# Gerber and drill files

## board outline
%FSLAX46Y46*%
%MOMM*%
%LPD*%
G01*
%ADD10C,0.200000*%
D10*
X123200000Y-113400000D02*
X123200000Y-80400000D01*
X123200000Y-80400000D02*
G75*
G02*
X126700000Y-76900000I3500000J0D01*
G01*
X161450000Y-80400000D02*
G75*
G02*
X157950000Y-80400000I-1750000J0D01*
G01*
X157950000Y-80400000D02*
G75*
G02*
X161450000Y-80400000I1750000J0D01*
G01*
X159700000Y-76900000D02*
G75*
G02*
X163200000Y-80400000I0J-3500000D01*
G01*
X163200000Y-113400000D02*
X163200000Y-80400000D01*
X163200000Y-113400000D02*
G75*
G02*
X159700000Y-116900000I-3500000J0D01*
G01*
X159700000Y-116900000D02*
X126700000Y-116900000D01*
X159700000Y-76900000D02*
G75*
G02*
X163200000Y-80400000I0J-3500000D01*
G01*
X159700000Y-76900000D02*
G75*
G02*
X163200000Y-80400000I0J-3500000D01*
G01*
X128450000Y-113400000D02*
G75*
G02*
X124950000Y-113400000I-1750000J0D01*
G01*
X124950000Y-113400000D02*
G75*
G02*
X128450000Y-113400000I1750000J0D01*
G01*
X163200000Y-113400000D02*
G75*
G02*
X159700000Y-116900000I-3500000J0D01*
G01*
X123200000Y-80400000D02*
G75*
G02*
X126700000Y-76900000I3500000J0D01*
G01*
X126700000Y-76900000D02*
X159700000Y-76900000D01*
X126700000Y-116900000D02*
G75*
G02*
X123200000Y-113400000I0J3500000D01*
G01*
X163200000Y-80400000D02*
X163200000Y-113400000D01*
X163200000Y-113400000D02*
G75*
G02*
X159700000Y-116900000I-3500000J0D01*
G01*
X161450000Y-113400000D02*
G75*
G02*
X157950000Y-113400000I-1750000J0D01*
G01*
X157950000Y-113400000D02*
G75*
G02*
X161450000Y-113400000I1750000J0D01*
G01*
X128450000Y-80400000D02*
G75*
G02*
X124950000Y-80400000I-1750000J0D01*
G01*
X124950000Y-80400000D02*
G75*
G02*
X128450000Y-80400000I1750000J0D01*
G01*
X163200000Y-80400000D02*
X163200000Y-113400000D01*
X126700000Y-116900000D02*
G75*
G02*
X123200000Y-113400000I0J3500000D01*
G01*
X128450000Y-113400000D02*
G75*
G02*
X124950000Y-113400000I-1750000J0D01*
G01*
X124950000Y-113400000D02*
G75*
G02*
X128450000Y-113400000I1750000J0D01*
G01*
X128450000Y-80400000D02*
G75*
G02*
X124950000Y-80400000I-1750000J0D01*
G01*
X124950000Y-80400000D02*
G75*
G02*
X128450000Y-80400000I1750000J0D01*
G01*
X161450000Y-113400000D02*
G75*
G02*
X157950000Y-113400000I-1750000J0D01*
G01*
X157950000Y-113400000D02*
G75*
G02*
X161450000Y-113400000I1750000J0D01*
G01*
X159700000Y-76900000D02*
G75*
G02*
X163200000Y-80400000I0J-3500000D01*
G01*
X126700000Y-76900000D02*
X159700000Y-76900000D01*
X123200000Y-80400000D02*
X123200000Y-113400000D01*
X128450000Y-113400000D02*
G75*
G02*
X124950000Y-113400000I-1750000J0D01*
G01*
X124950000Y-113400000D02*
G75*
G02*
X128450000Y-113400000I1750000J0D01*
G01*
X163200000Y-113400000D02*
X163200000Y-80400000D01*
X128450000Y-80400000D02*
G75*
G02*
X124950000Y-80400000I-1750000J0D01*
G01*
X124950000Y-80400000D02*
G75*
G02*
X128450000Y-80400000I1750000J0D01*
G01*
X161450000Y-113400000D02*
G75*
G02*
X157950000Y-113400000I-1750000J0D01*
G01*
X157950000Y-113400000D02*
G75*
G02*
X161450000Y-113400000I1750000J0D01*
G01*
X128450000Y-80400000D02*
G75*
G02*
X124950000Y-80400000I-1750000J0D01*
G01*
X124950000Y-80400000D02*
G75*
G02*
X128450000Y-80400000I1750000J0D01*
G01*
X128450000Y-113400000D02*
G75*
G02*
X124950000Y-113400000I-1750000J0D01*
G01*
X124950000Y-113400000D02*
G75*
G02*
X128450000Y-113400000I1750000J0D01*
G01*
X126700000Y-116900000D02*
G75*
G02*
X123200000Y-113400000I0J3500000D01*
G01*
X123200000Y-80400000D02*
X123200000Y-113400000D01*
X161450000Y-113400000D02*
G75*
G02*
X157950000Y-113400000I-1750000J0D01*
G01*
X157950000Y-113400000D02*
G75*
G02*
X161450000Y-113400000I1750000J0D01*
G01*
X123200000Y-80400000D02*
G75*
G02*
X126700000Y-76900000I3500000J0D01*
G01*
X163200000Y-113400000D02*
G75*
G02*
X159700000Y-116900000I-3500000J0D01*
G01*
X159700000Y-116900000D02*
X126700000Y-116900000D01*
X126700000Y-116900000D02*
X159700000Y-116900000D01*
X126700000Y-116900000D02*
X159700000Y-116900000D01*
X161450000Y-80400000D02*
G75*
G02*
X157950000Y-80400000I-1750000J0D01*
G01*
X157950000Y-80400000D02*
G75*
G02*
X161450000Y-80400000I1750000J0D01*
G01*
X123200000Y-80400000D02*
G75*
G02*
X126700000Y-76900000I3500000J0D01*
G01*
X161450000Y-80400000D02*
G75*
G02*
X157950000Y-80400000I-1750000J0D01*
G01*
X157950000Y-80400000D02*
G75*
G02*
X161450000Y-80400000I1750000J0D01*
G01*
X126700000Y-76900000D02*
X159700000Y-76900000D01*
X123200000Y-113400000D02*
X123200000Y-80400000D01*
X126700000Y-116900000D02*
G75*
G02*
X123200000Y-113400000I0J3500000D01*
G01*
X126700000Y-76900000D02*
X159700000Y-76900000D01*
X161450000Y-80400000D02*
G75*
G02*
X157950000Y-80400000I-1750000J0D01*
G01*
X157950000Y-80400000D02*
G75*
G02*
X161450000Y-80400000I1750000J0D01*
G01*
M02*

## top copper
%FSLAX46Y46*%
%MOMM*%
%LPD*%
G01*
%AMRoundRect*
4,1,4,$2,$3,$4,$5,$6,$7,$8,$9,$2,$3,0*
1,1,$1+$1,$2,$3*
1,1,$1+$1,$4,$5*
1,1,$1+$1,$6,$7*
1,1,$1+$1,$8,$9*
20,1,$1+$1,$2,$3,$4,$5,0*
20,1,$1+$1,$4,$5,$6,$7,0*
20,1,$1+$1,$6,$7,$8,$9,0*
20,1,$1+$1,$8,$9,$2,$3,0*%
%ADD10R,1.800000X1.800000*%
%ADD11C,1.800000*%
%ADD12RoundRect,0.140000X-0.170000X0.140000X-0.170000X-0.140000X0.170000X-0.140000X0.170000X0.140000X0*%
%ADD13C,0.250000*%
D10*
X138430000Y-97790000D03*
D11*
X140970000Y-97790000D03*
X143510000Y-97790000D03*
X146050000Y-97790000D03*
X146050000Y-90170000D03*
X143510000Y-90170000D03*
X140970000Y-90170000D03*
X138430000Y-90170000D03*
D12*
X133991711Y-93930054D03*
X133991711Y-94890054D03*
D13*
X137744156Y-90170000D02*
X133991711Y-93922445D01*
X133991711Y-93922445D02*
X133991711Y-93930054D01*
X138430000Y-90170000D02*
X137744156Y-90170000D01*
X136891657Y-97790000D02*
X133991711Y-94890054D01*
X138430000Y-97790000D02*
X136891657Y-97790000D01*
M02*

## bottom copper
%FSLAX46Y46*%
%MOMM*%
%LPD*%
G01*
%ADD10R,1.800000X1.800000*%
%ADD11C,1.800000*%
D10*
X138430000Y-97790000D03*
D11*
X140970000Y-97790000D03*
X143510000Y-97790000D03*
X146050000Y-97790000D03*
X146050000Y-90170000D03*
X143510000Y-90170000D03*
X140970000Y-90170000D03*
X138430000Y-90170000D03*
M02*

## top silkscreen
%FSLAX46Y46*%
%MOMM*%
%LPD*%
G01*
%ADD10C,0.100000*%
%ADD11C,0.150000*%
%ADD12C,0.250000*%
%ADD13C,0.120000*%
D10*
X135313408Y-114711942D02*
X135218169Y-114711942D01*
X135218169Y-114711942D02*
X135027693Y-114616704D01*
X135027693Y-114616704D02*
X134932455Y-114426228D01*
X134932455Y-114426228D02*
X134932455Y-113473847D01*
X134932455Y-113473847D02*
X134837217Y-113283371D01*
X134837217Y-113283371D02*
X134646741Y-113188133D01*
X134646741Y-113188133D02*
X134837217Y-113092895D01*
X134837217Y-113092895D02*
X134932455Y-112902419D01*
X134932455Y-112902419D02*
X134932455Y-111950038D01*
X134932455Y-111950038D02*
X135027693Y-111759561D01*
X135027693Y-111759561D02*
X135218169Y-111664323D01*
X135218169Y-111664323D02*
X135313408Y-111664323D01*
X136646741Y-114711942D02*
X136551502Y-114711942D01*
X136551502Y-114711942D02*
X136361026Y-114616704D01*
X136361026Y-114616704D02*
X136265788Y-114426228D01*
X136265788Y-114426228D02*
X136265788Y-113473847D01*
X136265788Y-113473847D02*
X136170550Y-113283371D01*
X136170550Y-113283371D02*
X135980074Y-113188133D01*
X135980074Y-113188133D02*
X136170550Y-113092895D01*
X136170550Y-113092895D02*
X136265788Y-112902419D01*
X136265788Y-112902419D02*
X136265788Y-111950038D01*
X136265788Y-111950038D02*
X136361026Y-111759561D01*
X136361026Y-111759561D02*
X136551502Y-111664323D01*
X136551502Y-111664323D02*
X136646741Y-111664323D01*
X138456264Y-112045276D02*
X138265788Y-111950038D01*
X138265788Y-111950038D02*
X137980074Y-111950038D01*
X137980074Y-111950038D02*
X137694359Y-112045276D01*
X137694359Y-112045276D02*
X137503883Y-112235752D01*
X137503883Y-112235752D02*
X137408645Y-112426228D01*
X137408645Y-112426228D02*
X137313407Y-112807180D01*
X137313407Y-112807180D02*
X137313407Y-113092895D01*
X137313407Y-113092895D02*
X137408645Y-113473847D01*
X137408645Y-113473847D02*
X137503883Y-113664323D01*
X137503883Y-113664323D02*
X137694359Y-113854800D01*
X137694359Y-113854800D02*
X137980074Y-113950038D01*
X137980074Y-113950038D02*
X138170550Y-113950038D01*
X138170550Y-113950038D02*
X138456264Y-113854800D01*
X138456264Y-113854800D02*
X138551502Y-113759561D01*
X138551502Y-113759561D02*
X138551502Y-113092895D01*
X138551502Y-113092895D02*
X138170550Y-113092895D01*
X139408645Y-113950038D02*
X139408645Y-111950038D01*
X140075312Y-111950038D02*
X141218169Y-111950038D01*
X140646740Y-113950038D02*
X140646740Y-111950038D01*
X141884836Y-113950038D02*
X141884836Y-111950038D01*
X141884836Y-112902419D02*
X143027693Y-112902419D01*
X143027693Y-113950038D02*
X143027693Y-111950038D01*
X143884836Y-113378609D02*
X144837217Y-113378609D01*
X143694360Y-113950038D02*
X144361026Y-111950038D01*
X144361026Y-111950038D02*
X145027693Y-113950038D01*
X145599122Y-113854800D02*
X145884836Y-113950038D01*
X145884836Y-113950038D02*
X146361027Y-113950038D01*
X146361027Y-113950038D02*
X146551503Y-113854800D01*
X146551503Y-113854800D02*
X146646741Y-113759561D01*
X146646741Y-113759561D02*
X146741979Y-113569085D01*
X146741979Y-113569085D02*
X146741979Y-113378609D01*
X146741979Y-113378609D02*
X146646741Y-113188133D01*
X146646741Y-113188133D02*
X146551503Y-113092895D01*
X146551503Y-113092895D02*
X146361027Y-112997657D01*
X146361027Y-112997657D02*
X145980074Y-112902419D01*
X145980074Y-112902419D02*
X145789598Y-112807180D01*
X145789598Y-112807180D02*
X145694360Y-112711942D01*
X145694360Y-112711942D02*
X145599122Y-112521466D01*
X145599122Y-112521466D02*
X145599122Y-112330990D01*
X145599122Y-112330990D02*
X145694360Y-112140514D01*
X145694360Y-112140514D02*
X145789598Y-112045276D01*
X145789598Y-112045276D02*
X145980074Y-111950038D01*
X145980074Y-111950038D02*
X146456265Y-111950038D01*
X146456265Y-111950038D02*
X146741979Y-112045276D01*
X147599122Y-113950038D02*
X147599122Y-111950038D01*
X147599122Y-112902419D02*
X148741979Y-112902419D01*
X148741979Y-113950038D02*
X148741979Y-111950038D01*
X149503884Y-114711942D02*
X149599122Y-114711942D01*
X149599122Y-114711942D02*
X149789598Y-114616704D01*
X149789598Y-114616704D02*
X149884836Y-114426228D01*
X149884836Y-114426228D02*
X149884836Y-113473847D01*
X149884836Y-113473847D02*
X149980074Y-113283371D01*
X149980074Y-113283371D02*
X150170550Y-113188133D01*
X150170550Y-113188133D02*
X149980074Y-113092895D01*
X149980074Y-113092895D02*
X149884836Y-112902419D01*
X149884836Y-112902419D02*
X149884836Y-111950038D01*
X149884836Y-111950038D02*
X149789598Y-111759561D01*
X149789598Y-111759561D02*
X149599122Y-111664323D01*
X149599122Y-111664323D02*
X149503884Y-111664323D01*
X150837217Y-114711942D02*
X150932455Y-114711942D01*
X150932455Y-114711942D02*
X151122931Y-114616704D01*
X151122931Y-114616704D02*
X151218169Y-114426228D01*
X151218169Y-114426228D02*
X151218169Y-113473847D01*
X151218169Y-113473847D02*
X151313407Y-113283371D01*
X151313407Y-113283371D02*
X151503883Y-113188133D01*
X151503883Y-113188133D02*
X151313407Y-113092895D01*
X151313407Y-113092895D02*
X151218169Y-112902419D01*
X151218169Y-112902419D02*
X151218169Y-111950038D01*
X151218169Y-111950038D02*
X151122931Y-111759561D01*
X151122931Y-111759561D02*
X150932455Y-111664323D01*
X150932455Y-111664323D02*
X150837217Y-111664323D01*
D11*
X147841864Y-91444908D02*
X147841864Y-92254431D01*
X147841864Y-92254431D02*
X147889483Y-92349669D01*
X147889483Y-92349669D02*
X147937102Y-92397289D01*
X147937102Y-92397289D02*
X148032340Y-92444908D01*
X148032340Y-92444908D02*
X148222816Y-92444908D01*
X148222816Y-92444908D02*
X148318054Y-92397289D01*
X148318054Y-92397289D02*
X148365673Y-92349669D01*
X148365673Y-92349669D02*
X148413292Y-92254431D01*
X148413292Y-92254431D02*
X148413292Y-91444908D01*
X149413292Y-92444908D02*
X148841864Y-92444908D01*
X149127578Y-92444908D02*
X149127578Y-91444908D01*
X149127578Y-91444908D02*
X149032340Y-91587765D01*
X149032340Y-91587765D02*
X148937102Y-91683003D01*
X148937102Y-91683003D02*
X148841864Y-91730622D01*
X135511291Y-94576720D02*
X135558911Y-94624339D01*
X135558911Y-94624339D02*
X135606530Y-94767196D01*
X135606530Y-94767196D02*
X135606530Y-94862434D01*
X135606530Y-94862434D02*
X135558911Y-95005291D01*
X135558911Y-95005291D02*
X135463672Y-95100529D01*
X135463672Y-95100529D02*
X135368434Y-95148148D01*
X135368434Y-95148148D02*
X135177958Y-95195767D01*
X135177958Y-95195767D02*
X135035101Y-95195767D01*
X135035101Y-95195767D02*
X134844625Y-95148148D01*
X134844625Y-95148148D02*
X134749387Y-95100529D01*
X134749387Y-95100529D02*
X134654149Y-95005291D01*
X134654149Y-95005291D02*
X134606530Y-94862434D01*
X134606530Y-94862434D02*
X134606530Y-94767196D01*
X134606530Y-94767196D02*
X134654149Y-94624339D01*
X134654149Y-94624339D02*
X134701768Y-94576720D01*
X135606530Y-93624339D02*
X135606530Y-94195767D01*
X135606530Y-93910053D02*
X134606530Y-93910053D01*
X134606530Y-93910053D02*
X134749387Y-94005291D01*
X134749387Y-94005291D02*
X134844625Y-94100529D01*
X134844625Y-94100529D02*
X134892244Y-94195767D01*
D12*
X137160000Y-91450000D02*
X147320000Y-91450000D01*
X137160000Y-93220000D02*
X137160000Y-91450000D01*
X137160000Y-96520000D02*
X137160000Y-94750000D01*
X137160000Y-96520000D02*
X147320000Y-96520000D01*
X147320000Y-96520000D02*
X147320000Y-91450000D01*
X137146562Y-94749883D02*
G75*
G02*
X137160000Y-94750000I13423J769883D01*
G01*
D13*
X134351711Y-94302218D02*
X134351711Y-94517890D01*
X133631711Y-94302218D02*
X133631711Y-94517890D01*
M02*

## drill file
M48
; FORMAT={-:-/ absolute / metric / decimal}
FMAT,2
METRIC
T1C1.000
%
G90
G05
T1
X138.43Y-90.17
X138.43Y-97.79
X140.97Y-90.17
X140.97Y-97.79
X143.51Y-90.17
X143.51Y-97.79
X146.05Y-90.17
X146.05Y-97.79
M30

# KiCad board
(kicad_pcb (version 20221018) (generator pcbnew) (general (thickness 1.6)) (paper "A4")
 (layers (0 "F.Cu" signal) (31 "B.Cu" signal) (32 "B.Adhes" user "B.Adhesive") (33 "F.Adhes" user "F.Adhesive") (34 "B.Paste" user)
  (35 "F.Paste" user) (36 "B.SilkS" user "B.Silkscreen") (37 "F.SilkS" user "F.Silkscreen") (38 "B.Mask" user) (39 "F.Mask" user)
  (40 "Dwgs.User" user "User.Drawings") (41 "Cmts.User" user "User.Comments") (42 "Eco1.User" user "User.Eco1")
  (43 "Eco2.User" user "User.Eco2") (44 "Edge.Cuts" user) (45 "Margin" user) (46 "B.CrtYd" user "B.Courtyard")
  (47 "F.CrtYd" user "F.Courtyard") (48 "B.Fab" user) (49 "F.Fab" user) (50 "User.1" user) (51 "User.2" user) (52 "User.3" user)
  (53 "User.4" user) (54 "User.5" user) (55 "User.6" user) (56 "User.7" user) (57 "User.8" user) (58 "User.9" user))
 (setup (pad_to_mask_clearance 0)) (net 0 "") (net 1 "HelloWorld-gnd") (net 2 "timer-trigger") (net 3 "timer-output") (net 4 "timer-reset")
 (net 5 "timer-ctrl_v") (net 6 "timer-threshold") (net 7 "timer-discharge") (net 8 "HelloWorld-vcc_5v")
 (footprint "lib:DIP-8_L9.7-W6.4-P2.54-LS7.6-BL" (layer "F.Cu") (at 142.24 93.98)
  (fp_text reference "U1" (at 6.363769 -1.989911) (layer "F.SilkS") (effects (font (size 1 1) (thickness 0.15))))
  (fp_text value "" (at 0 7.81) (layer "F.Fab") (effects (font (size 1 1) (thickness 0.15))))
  (fp_line (start -5.08 -2.53) (end 5.08 -2.53) (stroke (width 0.25) (type solid)) (layer "F.SilkS"))
  (fp_line (start -5.08 -0.76) (end -5.08 -2.53) (stroke (width 0.25) (type solid)) (layer "F.SilkS"))
  (fp_line (start -5.08 2.54) (end -5.08 0.77) (stroke (width 0.25) (type solid)) (layer "F.SilkS"))
  (fp_line (start -5.08 2.54) (end 5.08 2.54) (stroke (width 0.25) (type solid)) (layer "F.SilkS"))
  (fp_line (start 5.08 2.54) (end 5.08 -2.53) (stroke (width 0.25) (type solid)) (layer "F.SilkS"))
  (fp_arc (start -5.093438 0.769883) (mid -5.073311 -0.769971) (end -5.08 0.77) (stroke (width 0.25) (type solid)) (layer "F.SilkS"))
  (pad "1" thru_hole rect (at -3.81 3.81) (size 1.8 1.8) (drill 0.999998) (layers "*.Cu" "*.Mask") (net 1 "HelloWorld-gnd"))
  (pad "2" thru_hole circle (at -1.27 3.81) (size 1.8 1.8) (drill 0.999998) (layers "*.Cu" "*.Mask") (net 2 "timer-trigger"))
  (pad "3" thru_hole circle (at 1.27 3.81) (size 1.8 1.8) (drill 0.999998) (layers "*.Cu" "*.Mask") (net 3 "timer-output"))
  (pad "4" thru_hole circle (at 3.81 3.81) (size 1.8 1.8) (drill 0.999998) (layers "*.Cu" "*.Mask") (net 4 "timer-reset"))
  (pad "5" thru_hole circle (at 3.81 -3.81) (size 1.8 1.8) (drill 0.999998) (layers "*.Cu" "*.Mask") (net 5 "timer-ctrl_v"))
  (pad "6" thru_hole circle (at 1.27 -3.81) (size 1.8 1.8) (drill 0.999998) (layers "*.Cu" "*.Mask") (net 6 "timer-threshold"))
  (pad "7" thru_hole circle (at -1.27 -3.81) (size 1.8 1.8) (drill 0.999998) (layers "*.Cu" "*.Mask") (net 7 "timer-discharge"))
  (pad "8" thru_hole circle (at -3.81 -3.81) (size 1.8 1.8) (drill 0.999998) (layers "*.Cu" "*.Mask") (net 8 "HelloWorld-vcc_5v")))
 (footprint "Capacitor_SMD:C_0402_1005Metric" (layer "F.Cu") (at 133.991711 94.410054 -90)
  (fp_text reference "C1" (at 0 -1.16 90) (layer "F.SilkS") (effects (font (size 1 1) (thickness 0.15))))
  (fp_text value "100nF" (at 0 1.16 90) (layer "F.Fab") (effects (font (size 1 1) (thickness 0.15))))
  (fp_line (start -0.107836 -0.36) (end 0.107836 -0.36) (stroke (width 0.12) (type solid)) (layer "F.SilkS"))
  (fp_line (start -0.107836 0.36) (end 0.107836 0.36) (stroke (width 0.12) (type solid)) (layer "F.SilkS"))
  (pad "1" smd roundrect (at -0.48 0 270) (size 0.56 0.62) (layers "F.Cu" "F.Paste" "F.Mask") (roundrect_rratio 0.25)
   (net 8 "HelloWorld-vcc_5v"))
  (pad "2" smd roundrect (at 0.48 0 270) (size 0.56 0.62) (layers "F.Cu" "F.Paste" "F.Mask") (roundrect_rratio 0.25)
   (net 1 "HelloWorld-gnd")))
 (gr_line (start 123.2 113.4) (end 123.2 80.4) (stroke (width 0.2) (type solid)) (layer "Edge.Cuts"))
 (gr_arc (start 123.2 80.4) (mid 124.225126 77.925126) (end 126.7 76.9) (stroke (width 0.2) (type solid)) (layer "Edge.Cuts"))
 (gr_circle (center 159.7 80.4) (end 161.45 80.4) (stroke (width 0.2) (type solid)) (fill none) (layer "Edge.Cuts"))
 (gr_arc (start 159.7 76.9) (mid 162.174874 77.925126) (end 163.2 80.4) (stroke (width 0.2) (type solid)) (layer "Edge.Cuts"))
 (gr_line (start 163.2 113.4) (end 163.2 80.4) (stroke (width 0.2) (type solid)) (layer "Edge.Cuts"))
 (gr_arc (start 163.2 113.4) (mid 162.174874 115.874874) (end 159.7 116.9) (stroke (width 0.2) (type solid)) (layer "Edge.Cuts"))
 (gr_line (start 159.7 116.9) (end 126.7 116.9) (stroke (width 0.2) (type solid)) (layer "Edge.Cuts"))
 (gr_arc (start 159.7 76.9) (mid 162.174874 77.925126) (end 163.2 80.4) (stroke (width 0.2) (type solid)) (layer "Edge.Cuts"))
 (gr_arc (start 159.7 76.9) (mid 162.174874 77.925126) (end 163.2 80.4) (stroke (width 0.2) (type solid)) (layer "Edge.Cuts"))
 (gr_circle (center 126.7 113.4) (end 128.45 113.4) (stroke (width 0.2) (type solid)) (fill none) (layer "Edge.Cuts"))
 (gr_arc (start 163.2 113.4) (mid 162.174874 115.874874) (end 159.7 116.9) (stroke (width 0.2) (type solid)) (layer "Edge.Cuts"))
 (gr_arc (start 123.2 80.4) (mid 124.225126 77.925126) (end 126.7 76.9) (stroke (width 0.2) (type solid)) (layer "Edge.Cuts"))
 (gr_line (start 126.7 76.9) (end 159.7 76.9) (stroke (width 0.2) (type solid)) (layer "Edge.Cuts"))
 (gr_arc (start 126.7 116.9) (mid 124.225126 115.874874) (end 123.2 113.4) (stroke (width 0.2) (type solid)) (layer "Edge.Cuts"))
 (gr_line (start 163.2 80.4) (end 163.2 113.4) (stroke (width 0.2) (type solid)) (layer "Edge.Cuts"))
 (gr_arc (start 163.2 113.4) (mid 162.174874 115.874874) (end 159.7 116.9) (stroke (width 0.2) (type solid)) (layer "Edge.Cuts"))
 (gr_circle (center 159.7 113.4) (end 161.45 113.4) (stroke (width 0.2) (type solid)) (fill none) (layer "Edge.Cuts"))
 (gr_circle (center 126.7 80.4) (end 128.45 80.4) (stroke (width 0.2) (type solid)) (fill none) (layer "Edge.Cuts"))
 (gr_line (start 163.2 80.4) (end 163.2 113.4) (stroke (width 0.2) (type solid)) (layer "Edge.Cuts"))
 (gr_arc (start 126.7 116.9) (mid 124.225126 115.874874) (end 123.2 113.4) (stroke (width 0.2) (type solid)) (layer "Edge.Cuts"))
 (gr_circle (center 126.7 113.4) (end 128.45 113.4) (stroke (width 0.2) (type solid)) (fill none) (layer "Edge.Cuts"))
 (gr_circle (center 126.7 80.4) (end 128.45 80.4) (stroke (width 0.2) (type solid)) (fill none) (layer "Edge.Cuts"))
 (gr_circle (center 159.7 113.4) (end 161.45 113.4) (stroke (width 0.2) (type solid)) (fill none) (layer "Edge.Cuts"))
 (gr_arc (start 159.7 76.9) (mid 162.174874 77.925126) (end 163.2 80.4) (stroke (width 0.2) (type solid)) (layer "Edge.Cuts"))
 (gr_line (start 126.7 76.9) (end 159.7 76.9) (stroke (width 0.2) (type solid)) (layer "Edge.Cuts"))
 (gr_line (start 123.2 80.4) (end 123.2 113.4) (stroke (width 0.2) (type solid)) (layer "Edge.Cuts"))
 (gr_circle (center 126.7 113.4) (end 128.45 113.4) (stroke (width 0.2) (type solid)) (fill none) (layer "Edge.Cuts"))
 (gr_line (start 163.2 113.4) (end 163.2 80.4) (stroke (width 0.2) (type solid)) (layer "Edge.Cuts"))
 (gr_circle (center 126.7 80.4) (end 128.45 80.4) (stroke (width 0.2) (type solid)) (fill none) (layer "Edge.Cuts"))
 (gr_circle (center 159.7 113.4) (end 161.45 113.4) (stroke (width 0.2) (type solid)) (fill none) (layer "Edge.Cuts"))
 (gr_circle (center 126.7 80.4) (end 128.45 80.4) (stroke (width 0.2) (type solid)) (fill none) (layer "Edge.Cuts"))
 (gr_circle (center 126.7 113.4) (end 128.45 113.4) (stroke (width 0.2) (type solid)) (fill none) (layer "Edge.Cuts"))
 (gr_arc (start 126.7 116.9) (mid 124.225126 115.874874) (end 123.2 113.4) (stroke (width 0.2) (type solid)) (layer "Edge.Cuts"))
 (gr_line (start 123.2 80.4) (end 123.2 113.4) (stroke (width 0.2) (type solid)) (layer "Edge.Cuts"))
 (gr_circle (center 159.7 113.4) (end 161.45 113.4) (stroke (width 0.2) (type solid)) (fill none) (layer "Edge.Cuts"))
 (gr_arc (start 123.2 80.4) (mid 124.225126 77.925126) (end 126.7 76.9) (stroke (width 0.2) (type solid)) (layer "Edge.Cuts"))
 (gr_arc (start 163.2 113.4) (mid 162.174874 115.874874) (end 159.7 116.9) (stroke (width 0.2) (type solid)) (layer "Edge.Cuts"))
 (gr_line (start 159.7 116.9) (end 126.7 116.9) (stroke (width 0.2) (type solid)) (layer "Edge.Cuts"))
 (gr_line (start 126.7 116.9) (end 159.7 116.9) (stroke (width 0.2) (type solid)) (layer "Edge.Cuts"))
 (gr_line (start 126.7 116.9) (end 159.7 116.9) (stroke (width 0.2) (type solid)) (layer "Edge.Cuts"))
 (gr_circle (center 159.7 80.4) (end 161.45 80.4) (stroke (width 0.2) (type solid)) (fill none) (layer "Edge.Cuts"))
 (gr_arc (start 123.2 80.4) (mid 124.225126 77.925126) (end 126.7 76.9) (stroke (width 0.2) (type solid)) (layer "Edge.Cuts"))
 (gr_circle (center 159.7 80.4) (end 161.45 80.4) (stroke (width 0.2) (type solid)) (fill none) (layer "Edge.Cuts"))
 (gr_line (start 126.7 76.9) (end 159.7 76.9) (stroke (width 0.2) (type solid)) (layer "Edge.Cuts"))
 (gr_line (start 123.2 113.4) (end 123.2 80.4) (stroke (width 0.2) (type solid)) (layer "Edge.Cuts"))
 (gr_arc (start 126.7 116.9) (mid 124.225126 115.874874) (end 123.2 113.4) (stroke (width 0.2) (type solid)) (layer "Edge.Cuts"))
 (gr_line (start 126.7 76.9) (end 159.7 76.9) (stroke (width 0.2) (type solid)) (layer "Edge.Cuts"))
 (gr_circle (center 159.7 80.4) (end 161.45 80.4) (stroke (width 0.2) (type solid)) (fill none) (layer "Edge.Cuts"))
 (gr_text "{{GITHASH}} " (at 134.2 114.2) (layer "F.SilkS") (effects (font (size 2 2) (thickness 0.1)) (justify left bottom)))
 (segment (start 137.744156 90.17) (end 133.991711 93.922445) (width 0.25) (layer "F.Cu") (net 8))
 (segment (start 133.991711 93.922445) (end 133.991711 93.930054) (width 0.25) (layer "F.Cu") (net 8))
 (segment (start 138.43 90.17) (end 137.744156 90.17) (width 0.25) (layer "F.Cu") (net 8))
 (segment (start 136.891657 97.79) (end 133.991711 94.890054) (width 0.25) (layer "F.Cu") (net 1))
 (segment (start 138.43 97.79) (end 136.891657 97.79) (width 0.25) (layer "F.Cu") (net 1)))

